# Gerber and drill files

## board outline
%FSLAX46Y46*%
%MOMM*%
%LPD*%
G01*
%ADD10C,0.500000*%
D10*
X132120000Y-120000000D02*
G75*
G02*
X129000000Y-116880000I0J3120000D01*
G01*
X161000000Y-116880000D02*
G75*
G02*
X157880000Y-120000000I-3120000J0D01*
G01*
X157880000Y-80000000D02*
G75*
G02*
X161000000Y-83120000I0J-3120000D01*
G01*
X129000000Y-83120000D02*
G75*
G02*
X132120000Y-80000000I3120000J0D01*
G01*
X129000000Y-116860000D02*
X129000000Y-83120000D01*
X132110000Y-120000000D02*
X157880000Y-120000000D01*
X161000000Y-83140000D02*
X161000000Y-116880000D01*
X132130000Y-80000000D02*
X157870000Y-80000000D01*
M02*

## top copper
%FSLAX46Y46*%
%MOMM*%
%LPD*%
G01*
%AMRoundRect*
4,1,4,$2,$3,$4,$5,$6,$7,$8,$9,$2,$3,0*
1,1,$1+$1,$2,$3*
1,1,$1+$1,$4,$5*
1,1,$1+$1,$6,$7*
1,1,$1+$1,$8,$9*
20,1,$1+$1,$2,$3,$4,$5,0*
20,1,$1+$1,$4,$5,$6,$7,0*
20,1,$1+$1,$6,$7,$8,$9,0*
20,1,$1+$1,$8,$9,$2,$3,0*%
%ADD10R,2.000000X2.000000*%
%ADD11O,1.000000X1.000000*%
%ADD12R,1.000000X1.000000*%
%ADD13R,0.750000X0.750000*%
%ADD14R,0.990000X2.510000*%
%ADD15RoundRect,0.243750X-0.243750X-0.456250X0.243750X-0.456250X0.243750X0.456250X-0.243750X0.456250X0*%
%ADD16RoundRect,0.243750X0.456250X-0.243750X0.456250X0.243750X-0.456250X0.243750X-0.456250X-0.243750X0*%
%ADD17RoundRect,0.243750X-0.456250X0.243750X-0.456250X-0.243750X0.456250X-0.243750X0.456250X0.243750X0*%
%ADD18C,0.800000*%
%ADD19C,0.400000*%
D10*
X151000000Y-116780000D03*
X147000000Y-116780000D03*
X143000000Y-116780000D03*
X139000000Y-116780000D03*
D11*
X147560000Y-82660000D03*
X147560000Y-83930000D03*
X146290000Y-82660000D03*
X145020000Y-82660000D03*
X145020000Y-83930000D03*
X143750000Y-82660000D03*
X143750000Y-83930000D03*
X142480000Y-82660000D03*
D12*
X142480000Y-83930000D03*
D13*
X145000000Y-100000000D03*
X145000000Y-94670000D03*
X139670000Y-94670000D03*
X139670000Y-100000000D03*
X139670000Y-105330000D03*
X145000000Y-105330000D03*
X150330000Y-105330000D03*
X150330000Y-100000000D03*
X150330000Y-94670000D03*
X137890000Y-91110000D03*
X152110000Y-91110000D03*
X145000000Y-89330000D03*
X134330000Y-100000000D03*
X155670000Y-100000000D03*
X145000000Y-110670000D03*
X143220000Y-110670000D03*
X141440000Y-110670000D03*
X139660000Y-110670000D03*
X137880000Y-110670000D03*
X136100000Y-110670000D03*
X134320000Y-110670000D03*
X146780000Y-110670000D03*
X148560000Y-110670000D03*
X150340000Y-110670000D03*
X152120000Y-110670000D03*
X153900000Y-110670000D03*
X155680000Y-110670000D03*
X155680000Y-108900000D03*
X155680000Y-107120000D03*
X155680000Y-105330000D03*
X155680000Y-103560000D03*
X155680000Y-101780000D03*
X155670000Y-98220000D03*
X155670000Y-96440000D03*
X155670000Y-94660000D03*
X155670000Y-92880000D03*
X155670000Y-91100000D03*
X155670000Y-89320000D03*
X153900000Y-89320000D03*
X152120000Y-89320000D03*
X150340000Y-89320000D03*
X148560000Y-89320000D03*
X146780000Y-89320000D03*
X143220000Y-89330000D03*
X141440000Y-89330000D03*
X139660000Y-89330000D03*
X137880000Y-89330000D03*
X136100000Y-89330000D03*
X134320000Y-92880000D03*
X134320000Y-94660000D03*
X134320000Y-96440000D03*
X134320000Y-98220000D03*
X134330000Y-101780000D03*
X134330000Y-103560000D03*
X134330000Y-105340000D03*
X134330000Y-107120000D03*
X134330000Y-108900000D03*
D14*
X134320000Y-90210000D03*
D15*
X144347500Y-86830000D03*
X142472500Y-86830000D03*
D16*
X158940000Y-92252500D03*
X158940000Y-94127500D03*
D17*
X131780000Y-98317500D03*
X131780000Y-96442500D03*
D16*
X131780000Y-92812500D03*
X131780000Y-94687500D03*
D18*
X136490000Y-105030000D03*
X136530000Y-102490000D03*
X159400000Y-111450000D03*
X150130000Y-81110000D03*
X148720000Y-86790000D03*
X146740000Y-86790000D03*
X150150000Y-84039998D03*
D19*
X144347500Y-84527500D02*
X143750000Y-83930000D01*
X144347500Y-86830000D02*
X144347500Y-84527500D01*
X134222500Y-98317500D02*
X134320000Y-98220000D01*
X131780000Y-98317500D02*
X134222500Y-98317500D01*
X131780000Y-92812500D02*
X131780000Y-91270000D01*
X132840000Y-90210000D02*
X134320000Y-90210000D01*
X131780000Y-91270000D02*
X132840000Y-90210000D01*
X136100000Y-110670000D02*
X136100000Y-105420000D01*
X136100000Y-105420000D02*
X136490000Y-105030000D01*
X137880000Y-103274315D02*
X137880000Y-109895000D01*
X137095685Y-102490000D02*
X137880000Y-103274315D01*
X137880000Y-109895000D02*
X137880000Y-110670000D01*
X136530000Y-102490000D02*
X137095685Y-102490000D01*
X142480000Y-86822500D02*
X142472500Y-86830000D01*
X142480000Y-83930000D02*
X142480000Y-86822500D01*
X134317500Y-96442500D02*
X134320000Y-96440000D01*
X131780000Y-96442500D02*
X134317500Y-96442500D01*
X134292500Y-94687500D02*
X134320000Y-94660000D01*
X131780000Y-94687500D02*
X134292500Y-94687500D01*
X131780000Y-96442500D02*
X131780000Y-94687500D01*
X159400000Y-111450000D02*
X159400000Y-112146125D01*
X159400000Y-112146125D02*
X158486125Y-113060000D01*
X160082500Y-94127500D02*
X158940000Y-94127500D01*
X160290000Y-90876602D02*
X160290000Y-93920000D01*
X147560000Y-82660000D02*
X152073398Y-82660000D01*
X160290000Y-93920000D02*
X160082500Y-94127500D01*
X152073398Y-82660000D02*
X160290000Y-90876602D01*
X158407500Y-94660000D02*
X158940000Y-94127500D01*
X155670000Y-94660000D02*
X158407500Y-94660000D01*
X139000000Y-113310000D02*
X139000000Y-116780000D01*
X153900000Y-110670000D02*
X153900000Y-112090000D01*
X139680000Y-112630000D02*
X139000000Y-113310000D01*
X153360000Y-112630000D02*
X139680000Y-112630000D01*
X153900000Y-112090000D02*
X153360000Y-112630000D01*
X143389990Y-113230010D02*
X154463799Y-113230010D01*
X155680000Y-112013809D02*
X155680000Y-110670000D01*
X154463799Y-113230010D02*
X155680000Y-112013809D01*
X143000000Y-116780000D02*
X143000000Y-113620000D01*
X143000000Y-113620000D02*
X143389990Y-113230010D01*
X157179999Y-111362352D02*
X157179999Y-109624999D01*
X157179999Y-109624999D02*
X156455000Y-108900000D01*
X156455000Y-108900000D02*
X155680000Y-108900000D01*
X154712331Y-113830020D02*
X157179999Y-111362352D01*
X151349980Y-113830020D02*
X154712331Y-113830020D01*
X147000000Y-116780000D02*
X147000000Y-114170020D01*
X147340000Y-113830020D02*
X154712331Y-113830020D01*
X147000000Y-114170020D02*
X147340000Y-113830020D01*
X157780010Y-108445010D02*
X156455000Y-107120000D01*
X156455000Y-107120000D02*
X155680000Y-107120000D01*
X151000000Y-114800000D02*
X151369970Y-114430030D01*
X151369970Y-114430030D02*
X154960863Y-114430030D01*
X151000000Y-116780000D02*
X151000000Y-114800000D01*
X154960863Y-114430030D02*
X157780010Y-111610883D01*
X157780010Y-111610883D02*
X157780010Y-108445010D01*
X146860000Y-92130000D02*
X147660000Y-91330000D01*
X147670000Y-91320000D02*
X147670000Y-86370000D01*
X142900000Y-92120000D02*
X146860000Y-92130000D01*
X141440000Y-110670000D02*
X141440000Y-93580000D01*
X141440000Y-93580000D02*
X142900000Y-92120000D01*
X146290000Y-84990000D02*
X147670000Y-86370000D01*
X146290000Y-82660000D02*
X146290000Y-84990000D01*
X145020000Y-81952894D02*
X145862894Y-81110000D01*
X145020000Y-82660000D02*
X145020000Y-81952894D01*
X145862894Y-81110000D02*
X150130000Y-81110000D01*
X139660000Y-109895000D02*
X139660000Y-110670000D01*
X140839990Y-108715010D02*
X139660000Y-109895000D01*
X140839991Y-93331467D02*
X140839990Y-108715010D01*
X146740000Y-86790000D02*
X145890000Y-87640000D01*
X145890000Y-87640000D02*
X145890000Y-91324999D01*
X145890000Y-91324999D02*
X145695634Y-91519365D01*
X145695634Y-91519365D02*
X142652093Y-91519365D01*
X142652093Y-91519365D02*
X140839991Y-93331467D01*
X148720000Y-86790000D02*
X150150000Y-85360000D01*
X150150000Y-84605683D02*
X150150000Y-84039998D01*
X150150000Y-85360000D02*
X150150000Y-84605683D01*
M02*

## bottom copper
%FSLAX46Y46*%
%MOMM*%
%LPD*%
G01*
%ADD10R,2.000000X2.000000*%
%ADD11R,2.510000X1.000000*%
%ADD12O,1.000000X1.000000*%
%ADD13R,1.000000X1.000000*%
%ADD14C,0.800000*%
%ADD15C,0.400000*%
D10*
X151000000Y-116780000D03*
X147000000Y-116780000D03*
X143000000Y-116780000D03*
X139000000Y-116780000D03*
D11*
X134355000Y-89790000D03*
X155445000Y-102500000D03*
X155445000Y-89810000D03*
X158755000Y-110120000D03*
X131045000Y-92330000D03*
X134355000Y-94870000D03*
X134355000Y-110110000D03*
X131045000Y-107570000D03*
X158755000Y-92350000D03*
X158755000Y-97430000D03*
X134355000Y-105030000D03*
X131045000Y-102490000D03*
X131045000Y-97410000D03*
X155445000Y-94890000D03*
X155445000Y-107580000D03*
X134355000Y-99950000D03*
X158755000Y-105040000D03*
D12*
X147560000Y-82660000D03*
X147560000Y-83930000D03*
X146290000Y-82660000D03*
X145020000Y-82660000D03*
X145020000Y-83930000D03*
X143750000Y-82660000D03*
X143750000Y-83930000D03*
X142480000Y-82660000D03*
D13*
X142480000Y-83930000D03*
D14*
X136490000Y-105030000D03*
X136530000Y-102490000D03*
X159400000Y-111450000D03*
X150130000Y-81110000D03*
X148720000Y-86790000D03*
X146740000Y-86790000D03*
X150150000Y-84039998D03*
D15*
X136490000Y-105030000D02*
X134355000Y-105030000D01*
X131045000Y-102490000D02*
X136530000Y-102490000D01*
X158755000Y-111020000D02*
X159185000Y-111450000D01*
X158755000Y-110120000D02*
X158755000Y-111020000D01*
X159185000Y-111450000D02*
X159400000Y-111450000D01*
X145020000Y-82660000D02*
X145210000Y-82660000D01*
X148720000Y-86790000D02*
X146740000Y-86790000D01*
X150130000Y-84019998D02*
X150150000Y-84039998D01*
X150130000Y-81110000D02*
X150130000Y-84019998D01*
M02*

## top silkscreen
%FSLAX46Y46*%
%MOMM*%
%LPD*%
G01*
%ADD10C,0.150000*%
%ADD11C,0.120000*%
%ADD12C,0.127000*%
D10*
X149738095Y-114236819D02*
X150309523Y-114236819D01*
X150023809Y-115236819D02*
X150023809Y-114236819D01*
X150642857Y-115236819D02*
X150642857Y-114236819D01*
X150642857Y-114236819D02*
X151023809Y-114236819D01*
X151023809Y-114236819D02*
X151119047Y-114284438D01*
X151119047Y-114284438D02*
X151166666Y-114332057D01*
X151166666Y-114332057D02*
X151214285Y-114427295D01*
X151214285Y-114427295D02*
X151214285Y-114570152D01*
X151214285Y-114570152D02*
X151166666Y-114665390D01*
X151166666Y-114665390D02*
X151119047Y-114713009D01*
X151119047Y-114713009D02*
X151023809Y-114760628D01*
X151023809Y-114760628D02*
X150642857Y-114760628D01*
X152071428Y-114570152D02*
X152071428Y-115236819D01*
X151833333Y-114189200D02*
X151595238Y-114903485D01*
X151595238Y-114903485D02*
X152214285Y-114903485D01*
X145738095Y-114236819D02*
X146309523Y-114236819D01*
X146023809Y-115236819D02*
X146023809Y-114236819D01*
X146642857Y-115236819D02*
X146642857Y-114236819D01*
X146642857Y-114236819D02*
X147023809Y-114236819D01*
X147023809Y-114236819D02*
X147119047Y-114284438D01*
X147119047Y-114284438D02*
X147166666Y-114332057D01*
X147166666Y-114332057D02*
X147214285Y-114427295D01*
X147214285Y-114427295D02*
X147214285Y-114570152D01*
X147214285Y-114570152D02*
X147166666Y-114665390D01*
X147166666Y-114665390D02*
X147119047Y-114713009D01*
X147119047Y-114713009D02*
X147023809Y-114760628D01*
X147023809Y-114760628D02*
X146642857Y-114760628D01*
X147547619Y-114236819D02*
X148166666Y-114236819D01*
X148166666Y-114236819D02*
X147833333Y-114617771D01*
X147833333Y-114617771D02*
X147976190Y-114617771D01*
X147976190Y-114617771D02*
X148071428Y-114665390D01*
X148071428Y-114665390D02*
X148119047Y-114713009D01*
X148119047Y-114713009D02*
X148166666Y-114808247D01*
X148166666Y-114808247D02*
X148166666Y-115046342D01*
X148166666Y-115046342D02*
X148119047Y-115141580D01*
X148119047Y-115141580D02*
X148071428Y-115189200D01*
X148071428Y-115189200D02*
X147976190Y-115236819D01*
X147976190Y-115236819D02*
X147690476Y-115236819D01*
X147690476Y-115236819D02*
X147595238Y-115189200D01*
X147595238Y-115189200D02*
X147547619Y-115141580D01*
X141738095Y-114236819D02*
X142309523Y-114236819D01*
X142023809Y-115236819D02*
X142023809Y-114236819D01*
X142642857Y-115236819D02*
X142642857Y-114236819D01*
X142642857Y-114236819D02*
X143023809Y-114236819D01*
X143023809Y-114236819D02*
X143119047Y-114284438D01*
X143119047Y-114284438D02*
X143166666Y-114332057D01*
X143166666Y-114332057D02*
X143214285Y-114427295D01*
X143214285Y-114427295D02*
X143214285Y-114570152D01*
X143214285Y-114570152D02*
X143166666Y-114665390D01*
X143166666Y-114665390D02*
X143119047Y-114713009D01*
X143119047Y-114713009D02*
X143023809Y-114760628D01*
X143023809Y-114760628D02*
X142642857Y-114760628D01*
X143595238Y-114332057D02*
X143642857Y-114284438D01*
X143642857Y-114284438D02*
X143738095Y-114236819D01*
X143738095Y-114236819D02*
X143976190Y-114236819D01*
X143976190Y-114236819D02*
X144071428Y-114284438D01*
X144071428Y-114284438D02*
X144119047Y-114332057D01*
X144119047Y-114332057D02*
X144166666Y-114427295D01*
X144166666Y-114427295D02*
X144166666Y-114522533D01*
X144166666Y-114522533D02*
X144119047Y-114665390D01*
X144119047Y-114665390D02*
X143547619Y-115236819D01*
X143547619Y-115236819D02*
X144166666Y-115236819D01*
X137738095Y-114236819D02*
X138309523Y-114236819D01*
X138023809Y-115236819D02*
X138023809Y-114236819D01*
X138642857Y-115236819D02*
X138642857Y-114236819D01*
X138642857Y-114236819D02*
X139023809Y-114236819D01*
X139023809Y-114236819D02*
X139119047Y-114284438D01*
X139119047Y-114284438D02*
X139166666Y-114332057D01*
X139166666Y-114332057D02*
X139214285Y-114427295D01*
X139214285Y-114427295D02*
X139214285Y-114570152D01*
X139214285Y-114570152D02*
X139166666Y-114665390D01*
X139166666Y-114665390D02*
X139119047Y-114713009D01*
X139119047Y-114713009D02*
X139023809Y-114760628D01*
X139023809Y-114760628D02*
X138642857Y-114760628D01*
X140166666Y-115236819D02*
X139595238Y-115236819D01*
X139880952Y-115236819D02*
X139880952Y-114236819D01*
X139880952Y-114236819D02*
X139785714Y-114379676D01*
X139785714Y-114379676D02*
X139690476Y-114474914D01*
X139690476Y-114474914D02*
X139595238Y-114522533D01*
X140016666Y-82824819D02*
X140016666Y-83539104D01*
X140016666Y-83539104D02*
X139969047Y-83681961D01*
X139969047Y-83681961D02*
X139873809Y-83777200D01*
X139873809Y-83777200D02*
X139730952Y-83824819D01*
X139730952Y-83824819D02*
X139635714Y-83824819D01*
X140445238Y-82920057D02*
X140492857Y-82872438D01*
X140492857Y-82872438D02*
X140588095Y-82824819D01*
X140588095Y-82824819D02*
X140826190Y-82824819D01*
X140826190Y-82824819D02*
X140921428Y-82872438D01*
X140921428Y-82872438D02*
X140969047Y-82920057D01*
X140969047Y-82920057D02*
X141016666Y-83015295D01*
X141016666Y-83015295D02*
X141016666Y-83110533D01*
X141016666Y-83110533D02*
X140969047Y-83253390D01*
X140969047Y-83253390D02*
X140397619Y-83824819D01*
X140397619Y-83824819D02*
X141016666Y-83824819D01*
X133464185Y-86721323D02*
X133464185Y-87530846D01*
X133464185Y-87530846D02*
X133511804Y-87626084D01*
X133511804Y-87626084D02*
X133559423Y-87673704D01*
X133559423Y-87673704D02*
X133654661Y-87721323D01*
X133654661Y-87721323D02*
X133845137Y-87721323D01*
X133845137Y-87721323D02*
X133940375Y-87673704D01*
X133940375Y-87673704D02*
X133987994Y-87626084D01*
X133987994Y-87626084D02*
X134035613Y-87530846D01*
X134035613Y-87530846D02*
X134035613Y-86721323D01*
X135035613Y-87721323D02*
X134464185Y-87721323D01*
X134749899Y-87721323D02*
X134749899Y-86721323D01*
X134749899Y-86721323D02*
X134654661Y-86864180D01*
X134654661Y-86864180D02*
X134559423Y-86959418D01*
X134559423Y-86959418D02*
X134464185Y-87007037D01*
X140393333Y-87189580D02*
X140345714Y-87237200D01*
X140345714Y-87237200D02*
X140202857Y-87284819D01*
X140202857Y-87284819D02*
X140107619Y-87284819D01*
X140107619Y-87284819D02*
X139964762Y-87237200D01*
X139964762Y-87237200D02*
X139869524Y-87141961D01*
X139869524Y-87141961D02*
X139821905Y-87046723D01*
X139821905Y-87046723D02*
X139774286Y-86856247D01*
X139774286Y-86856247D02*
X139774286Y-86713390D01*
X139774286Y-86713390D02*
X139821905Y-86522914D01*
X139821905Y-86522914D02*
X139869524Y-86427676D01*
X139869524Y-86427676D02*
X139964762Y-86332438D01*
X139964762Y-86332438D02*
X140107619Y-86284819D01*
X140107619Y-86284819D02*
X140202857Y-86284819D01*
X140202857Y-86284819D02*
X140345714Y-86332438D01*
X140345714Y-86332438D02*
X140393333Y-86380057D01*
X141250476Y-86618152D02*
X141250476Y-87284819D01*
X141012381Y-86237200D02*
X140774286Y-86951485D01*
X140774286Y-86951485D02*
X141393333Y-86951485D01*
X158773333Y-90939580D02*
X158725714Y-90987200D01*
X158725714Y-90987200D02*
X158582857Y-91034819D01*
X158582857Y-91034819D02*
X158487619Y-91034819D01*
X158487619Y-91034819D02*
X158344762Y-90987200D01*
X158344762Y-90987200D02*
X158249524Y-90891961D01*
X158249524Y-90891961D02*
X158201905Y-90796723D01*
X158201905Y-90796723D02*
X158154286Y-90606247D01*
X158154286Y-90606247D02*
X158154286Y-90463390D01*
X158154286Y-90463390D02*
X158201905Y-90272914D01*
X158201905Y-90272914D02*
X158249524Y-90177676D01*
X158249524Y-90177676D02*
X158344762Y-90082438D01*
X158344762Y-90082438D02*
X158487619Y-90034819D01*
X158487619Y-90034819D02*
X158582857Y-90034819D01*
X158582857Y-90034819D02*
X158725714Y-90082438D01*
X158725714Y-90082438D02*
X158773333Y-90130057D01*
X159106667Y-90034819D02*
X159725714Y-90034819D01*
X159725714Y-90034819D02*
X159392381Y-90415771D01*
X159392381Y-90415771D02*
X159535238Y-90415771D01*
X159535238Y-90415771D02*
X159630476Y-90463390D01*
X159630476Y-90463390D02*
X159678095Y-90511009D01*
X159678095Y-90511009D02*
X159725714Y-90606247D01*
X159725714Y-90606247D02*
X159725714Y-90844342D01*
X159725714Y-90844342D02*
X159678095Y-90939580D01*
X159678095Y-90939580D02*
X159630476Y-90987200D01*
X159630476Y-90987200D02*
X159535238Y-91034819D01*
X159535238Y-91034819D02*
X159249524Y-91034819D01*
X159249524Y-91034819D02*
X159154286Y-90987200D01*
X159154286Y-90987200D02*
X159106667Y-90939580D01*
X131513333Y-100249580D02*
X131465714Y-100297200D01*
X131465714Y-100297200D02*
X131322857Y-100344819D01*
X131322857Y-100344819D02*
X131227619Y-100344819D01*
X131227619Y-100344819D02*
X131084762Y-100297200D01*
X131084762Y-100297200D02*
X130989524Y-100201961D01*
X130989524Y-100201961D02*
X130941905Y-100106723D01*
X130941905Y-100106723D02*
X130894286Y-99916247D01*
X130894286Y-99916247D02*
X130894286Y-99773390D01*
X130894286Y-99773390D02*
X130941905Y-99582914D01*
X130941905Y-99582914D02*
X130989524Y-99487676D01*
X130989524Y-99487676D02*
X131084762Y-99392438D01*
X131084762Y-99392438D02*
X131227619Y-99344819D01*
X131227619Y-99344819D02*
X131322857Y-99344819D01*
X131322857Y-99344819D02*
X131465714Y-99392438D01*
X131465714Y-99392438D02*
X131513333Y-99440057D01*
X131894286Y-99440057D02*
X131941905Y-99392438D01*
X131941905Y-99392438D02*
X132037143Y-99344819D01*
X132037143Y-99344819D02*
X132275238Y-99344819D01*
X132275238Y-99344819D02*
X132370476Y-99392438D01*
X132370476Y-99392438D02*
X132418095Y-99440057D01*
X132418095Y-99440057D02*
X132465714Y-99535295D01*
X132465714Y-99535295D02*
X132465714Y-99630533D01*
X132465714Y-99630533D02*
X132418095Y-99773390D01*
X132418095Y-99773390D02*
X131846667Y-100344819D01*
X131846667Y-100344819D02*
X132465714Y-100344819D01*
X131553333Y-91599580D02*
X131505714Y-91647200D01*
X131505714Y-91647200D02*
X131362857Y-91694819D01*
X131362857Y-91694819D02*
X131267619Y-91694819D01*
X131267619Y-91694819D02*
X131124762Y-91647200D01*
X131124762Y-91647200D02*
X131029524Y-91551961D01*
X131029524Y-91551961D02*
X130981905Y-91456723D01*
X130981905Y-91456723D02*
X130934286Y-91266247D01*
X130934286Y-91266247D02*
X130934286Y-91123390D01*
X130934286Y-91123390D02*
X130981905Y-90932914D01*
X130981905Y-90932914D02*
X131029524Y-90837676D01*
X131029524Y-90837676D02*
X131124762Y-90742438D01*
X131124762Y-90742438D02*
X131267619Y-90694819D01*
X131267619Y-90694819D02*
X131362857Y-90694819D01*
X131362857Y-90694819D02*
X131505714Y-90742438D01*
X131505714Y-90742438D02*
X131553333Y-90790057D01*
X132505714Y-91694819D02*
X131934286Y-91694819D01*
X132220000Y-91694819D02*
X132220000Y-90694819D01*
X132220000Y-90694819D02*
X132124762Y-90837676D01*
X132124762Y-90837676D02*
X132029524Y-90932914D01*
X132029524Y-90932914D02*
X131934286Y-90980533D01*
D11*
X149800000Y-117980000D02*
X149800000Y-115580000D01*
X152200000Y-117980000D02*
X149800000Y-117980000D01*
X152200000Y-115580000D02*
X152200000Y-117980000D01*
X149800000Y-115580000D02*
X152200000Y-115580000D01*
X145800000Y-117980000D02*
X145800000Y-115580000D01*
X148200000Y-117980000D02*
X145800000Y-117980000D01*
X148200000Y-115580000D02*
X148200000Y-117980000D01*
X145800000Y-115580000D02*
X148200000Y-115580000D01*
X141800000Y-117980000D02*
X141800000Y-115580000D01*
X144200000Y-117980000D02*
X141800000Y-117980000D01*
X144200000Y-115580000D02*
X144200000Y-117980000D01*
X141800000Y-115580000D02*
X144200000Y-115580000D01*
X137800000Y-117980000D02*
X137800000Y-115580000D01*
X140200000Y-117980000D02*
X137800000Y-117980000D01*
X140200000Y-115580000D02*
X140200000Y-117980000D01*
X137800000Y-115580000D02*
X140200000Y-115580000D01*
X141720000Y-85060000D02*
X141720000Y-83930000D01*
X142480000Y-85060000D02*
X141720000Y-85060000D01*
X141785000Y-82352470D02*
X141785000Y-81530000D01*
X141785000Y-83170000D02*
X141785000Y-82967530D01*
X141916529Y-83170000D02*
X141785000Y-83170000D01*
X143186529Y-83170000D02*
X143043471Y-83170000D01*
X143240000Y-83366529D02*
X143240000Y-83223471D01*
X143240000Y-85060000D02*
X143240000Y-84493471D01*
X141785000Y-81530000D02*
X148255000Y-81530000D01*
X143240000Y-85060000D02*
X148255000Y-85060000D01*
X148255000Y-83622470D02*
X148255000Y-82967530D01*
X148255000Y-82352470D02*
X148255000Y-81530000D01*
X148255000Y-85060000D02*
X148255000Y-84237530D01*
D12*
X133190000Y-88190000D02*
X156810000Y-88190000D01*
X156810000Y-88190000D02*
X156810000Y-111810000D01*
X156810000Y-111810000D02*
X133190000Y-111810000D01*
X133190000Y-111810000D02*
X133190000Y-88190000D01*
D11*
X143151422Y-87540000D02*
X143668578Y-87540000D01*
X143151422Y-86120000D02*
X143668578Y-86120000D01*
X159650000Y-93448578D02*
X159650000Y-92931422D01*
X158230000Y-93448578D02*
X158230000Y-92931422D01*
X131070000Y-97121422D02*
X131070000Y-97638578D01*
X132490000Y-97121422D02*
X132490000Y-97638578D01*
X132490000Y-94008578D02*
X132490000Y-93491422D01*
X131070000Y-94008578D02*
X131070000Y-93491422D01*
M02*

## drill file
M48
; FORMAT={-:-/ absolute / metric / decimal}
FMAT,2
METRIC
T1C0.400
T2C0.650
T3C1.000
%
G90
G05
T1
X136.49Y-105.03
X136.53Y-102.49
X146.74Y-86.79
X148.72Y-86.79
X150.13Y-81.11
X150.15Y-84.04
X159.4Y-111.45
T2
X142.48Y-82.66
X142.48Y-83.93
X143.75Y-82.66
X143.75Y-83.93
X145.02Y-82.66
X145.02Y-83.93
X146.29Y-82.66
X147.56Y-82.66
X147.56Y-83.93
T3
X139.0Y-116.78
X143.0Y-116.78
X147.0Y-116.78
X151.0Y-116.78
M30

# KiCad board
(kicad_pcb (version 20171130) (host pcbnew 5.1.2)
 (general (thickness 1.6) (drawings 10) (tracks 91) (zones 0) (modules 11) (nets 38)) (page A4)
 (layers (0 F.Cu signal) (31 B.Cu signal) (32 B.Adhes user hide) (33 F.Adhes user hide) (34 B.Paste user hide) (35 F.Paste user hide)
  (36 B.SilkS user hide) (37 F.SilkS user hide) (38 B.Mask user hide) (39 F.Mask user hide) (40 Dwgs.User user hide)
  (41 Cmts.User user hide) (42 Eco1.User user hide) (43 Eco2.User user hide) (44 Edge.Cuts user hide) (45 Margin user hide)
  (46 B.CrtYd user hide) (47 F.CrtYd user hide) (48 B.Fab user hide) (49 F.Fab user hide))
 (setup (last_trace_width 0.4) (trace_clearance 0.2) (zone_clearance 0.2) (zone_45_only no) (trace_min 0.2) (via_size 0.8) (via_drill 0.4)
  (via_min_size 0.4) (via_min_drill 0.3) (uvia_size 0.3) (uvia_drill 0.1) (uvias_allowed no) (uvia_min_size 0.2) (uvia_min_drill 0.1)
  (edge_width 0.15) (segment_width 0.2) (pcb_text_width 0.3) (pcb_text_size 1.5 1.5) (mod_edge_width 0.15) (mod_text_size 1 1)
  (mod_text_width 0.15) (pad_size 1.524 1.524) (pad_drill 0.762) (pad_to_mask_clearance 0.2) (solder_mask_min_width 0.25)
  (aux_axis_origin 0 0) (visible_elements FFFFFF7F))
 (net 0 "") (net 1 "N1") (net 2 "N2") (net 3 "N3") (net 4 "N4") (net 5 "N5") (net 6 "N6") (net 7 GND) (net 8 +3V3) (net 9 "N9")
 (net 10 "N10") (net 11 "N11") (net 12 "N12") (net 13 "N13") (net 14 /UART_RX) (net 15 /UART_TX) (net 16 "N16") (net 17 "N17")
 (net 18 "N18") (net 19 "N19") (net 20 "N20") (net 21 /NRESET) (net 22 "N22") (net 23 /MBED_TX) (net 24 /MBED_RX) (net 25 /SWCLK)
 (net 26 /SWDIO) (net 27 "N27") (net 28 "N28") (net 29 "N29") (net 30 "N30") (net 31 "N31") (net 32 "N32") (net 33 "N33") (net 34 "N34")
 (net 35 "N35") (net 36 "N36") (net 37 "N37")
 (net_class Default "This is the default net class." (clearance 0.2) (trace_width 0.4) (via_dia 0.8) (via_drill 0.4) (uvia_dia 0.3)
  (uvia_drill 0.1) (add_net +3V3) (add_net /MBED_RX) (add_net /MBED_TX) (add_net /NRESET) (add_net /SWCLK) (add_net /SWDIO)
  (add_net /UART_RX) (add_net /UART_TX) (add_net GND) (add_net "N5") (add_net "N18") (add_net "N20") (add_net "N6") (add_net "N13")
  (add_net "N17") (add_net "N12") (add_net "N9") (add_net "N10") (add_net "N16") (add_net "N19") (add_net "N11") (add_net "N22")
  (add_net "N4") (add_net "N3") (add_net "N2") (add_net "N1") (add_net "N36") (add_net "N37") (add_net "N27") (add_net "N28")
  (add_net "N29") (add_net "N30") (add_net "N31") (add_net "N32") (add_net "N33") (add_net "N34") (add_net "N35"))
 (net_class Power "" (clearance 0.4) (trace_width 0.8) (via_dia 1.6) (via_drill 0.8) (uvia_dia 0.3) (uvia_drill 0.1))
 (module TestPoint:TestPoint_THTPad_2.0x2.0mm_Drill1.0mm (layer F.Cu) (at 151 116.78)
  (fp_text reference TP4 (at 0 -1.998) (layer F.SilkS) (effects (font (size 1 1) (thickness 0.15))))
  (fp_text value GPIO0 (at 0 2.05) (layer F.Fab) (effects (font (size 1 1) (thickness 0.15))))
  (fp_line (start -1.2 1.2) (end -1.2 -1.2) (layer F.SilkS) (width 0.12))
  (fp_line (start 1.2 1.2) (end -1.2 1.2) (layer F.SilkS) (width 0.12))
  (fp_line (start 1.2 -1.2) (end 1.2 1.2) (layer F.SilkS) (width 0.12))
  (fp_line (start -1.2 -1.2) (end 1.2 -1.2) (layer F.SilkS) (width 0.12))
  (pad 1 thru_hole rect (at 0 0) (size 2 2) (drill 1) (layers *.Cu *.Mask) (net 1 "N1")))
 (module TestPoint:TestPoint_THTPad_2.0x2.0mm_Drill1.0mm (layer F.Cu) (at 147 116.78)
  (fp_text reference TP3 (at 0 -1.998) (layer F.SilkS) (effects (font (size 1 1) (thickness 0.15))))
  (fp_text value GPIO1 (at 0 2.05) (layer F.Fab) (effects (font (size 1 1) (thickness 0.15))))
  (fp_line (start -1.2 1.2) (end -1.2 -1.2) (layer F.SilkS) (width 0.12))
  (fp_line (start 1.2 1.2) (end -1.2 1.2) (layer F.SilkS) (width 0.12))
  (fp_line (start 1.2 -1.2) (end 1.2 1.2) (layer F.SilkS) (width 0.12))
  (fp_line (start -1.2 -1.2) (end 1.2 -1.2) (layer F.SilkS) (width 0.12))
  (pad 1 thru_hole rect (at 0 0) (size 2 2) (drill 1) (layers *.Cu *.Mask) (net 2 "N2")))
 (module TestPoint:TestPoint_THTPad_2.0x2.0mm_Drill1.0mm (layer F.Cu) (at 143 116.78)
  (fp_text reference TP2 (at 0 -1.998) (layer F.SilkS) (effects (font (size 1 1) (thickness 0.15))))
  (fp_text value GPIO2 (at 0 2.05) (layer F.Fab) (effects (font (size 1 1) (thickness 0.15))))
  (fp_line (start -1.2 1.2) (end -1.2 -1.2) (layer F.SilkS) (width 0.12))
  (fp_line (start 1.2 1.2) (end -1.2 1.2) (layer F.SilkS) (width 0.12))
  (fp_line (start 1.2 -1.2) (end 1.2 1.2) (layer F.SilkS) (width 0.12))
  (fp_line (start -1.2 -1.2) (end 1.2 -1.2) (layer F.SilkS) (width 0.12))
  (pad 1 thru_hole rect (at 0 0) (size 2 2) (drill 1) (layers *.Cu *.Mask) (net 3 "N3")))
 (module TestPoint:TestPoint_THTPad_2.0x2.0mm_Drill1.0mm (layer F.Cu) (at 139 116.78)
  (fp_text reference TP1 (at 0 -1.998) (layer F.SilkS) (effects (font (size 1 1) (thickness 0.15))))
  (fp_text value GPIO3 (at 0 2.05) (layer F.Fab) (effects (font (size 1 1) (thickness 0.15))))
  (fp_line (start -1.2 1.2) (end -1.2 -1.2) (layer F.SilkS) (width 0.12))
  (fp_line (start 1.2 1.2) (end -1.2 1.2) (layer F.SilkS) (width 0.12))
  (fp_line (start 1.2 -1.2) (end 1.2 1.2) (layer F.SilkS) (width 0.12))
  (fp_line (start -1.2 -1.2) (end 1.2 -1.2) (layer F.SilkS) (width 0.12))
  (pad 1 thru_hole rect (at 0 0) (size 2 2) (drill 1) (layers *.Cu *.Mask) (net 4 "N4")))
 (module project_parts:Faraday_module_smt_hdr (layer B.Cu) (at 145 100 180)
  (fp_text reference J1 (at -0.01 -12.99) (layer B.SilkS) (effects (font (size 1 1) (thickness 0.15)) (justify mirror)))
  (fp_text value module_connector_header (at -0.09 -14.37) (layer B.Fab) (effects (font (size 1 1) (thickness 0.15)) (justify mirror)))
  (pad 1 smd rect (at 10.645 10.21 180) (size 2.51 1) (layers B.Cu B.Paste B.Mask) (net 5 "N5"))
  (pad 13 smd rect (at -10.445 -2.5 180) (size 2.51 1) (layers B.Cu B.Paste B.Mask) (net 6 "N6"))
  (pad 17 smd rect (at -10.445 10.19 180) (size 2.51 1) (layers B.Cu B.Paste B.Mask) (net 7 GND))
  (pad 10 smd rect (at -13.755 -10.12 180) (size 2.51 1) (layers B.Cu B.Paste B.Mask) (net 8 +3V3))
  (pad 2 smd rect (at 13.955 7.67 180) (size 2.51 1) (layers B.Cu B.Paste B.Mask) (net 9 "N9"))
  (pad 3 smd rect (at 10.645 5.13 180) (size 2.51 1) (layers B.Cu B.Paste B.Mask) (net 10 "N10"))
  (pad 9 smd rect (at 10.645 -10.11 180) (size 2.51 1) (layers B.Cu B.Paste B.Mask) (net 7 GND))
  (pad 8 smd rect (at 13.955 -7.57 180) (size 2.51 1) (layers B.Cu B.Paste B.Mask) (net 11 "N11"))
  (pad 16 smd rect (at -13.755 7.65 180) (size 2.51 1) (layers B.Cu B.Paste B.Mask) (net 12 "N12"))
  (pad 14 smd rect (at -13.755 2.57 180) (size 2.51 1) (layers B.Cu B.Paste B.Mask) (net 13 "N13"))
  (pad 7 smd rect (at 10.645 -5.03 180) (size 2.51 1) (layers B.Cu B.Paste B.Mask) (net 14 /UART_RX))
  (pad 6 smd rect (at 13.955 -2.49 180) (size 2.51 1) (layers B.Cu B.Paste B.Mask) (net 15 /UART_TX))
  (pad 4 smd rect (at 13.955 2.59 180) (size 2.51 1) (layers B.Cu B.Paste B.Mask) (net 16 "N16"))
  (pad 15 smd rect (at -10.445 5.11 180) (size 2.51 1) (layers B.Cu B.Paste B.Mask) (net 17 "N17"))
  (pad 11 smd rect (at -10.445 -7.58 180) (size 2.51 1) (layers B.Cu B.Paste B.Mask) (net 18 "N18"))
  (pad 5 smd rect (at 10.645 0.05 180) (size 2.51 1) (layers B.Cu B.Paste B.Mask) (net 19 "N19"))
  (pad 12 smd rect (at -13.755 -5.04 180) (size 2.51 1) (layers B.Cu B.Paste B.Mask) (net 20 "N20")))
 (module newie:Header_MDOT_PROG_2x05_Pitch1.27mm (layer F.Cu) (at 142.48 83.93 90)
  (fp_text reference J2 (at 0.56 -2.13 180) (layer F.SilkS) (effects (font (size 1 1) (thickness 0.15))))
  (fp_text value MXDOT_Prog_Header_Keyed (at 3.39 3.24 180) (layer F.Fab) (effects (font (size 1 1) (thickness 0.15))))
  (fp_line (start -1.13 -0.76) (end 0 -0.76) (layer F.SilkS) (width 0.12))
  (fp_line (start -1.13 0) (end -1.13 -0.76) (layer F.SilkS) (width 0.12))
  (fp_line (start 1.57753 -0.695) (end 2.4 -0.695) (layer F.SilkS) (width 0.12))
  (fp_line (start 0.76 -0.695) (end 0.96247 -0.695) (layer F.SilkS) (width 0.12))
  (fp_line (start 0.76 -0.563471) (end 0.76 -0.695) (layer F.SilkS) (width 0.12))
  (fp_line (start 0.76 0.706529) (end 0.76 0.563471) (layer F.SilkS) (width 0.12))
  (fp_line (start 0.563471 0.76) (end 0.706529 0.76) (layer F.SilkS) (width 0.12))
  (fp_line (start -1.13 0.76) (end -0.563471 0.76) (layer F.SilkS) (width 0.12))
  (fp_line (start 2.4 -0.695) (end 2.4 5.775) (layer F.SilkS) (width 0.12))
  (fp_line (start -1.13 0.76) (end -1.13 5.775) (layer F.SilkS) (width 0.12))
  (fp_line (start 0.30753 5.775) (end 0.96247 5.775) (layer F.SilkS) (width 0.12))
  (fp_line (start 1.57753 5.775) (end 2.4 5.775) (layer F.SilkS) (width 0.12))
  (fp_line (start -1.13 5.775) (end -0.30753 5.775) (layer F.SilkS) (width 0.12))
  (pad 10 thru_hole oval (at 1.27 5.08 90) (size 1 1) (drill 0.65) (layers *.Cu *.Mask) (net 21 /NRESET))
  (pad 9 thru_hole oval (at 0 5.08 90) (size 1 1) (drill 0.65) (layers *.Cu *.Mask) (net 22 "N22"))
  (pad 8 thru_hole oval (at 1.27 3.81 90) (size 1 1) (drill 0.65) (layers *.Cu *.Mask) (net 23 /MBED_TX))
  (pad 6 thru_hole oval (at 1.27 2.54 90) (size 1 1) (drill 0.65) (layers *.Cu *.Mask) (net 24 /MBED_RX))
  (pad 5 thru_hole oval (at 0 2.54 90) (size 1 1) (drill 0.65) (layers *.Cu *.Mask) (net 7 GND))
  (pad 4 thru_hole oval (at 1.27 1.27 90) (size 1 1) (drill 0.65) (layers *.Cu *.Mask) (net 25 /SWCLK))
  (pad 3 thru_hole oval (at 0 1.27 90) (size 1 1) (drill 0.65) (layers *.Cu *.Mask) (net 7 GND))
  (pad 2 thru_hole oval (at 1.27 0 90) (size 1 1) (drill 0.65) (layers *.Cu *.Mask) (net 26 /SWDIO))
  (pad 1 thru_hole rect (at 0 0 90) (size 1 1) (drill 0.65) (layers *.Cu *.Mask) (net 8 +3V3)))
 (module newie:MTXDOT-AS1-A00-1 (layer F.Cu) (at 145 100)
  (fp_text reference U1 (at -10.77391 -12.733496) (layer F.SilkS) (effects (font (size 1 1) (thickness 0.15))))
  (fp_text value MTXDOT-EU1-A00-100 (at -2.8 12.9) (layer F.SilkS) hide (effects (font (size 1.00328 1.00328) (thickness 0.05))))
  (fp_line (start -11.81 -11.81) (end 11.81 -11.81) (layer F.SilkS) (width 0.127))
  (fp_line (start 11.81 -11.81) (end 11.81 11.81) (layer F.SilkS) (width 0.127))
  (fp_line (start 11.81 11.81) (end -11.81 11.81) (layer F.SilkS) (width 0.127))
  (fp_line (start -11.81 11.81) (end -11.81 -11.81) (layer F.SilkS) (width 0.127))
  (pad 54 smd rect (at 0 0) (size 0.75 0.75) (layers F.Cu F.Paste F.Mask) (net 7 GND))
  (pad 51 smd rect (at 0 -5.33) (size 0.75 0.75) (layers F.Cu F.Paste F.Mask) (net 7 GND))
  (pad 50 smd rect (at -5.33 -5.33) (size 0.75 0.75) (layers F.Cu F.Paste F.Mask) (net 7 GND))
  (pad 53 smd rect (at -5.33 0) (size 0.75 0.75) (layers F.Cu F.Paste F.Mask) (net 7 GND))
  (pad 56 smd rect (at -5.33 5.33) (size 0.75 0.75) (layers F.Cu F.Paste F.Mask) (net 7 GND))
  (pad 57 smd rect (at 0 5.33) (size 0.75 0.75) (layers F.Cu F.Paste F.Mask) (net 7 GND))
  (pad 58 smd rect (at 5.33 5.33) (size 0.75 0.75) (layers F.Cu F.Paste F.Mask) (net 7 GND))
  (pad 55 smd rect (at 5.33 0) (size 0.75 0.75) (layers F.Cu F.Paste F.Mask) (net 7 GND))
  (pad 52 smd rect (at 5.33 -5.33) (size 0.75 0.75) (layers F.Cu F.Paste F.Mask) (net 7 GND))
  (pad 49 smd rect (at -7.11 -8.89) (size 0.75 0.75) (layers F.Cu F.Paste F.Mask) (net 7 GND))
  (pad 48 smd rect (at 7.11 -8.89) (size 0.75 0.75) (layers F.Cu F.Paste F.Mask) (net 7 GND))
  (pad 42 smd rect (at 0 -10.67) (size 0.75 0.75) (layers F.Cu F.Paste F.Mask) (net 7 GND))
  (pad 6 smd rect (at -10.67 0) (size 0.75 0.75) (layers F.Cu F.Paste F.Mask))
  (pad 30 smd rect (at 10.67 0) (size 0.75 0.75) (layers F.Cu F.Paste F.Mask) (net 26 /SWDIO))
  (pad 18 smd rect (at 0 10.67) (size 0.75 0.75) (layers F.Cu F.Paste F.Mask))
  (pad 17 smd rect (at -1.78 10.67) (size 0.75 0.75) (layers F.Cu F.Paste F.Mask) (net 7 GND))
  (pad 16 smd rect (at -3.56 10.67) (size 0.75 0.75) (layers F.Cu F.Paste F.Mask) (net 23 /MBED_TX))
  (pad 15 smd rect (at -5.34 10.67) (size 0.75 0.75) (layers F.Cu F.Paste F.Mask) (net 24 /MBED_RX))
  (pad 14 smd rect (at -7.12 10.67) (size 0.75 0.75) (layers F.Cu F.Paste F.Mask) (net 15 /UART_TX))
  (pad 13 smd rect (at -8.9 10.67) (size 0.75 0.75) (layers F.Cu F.Paste F.Mask) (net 14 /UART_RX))
  (pad 12 smd rect (at -10.68 10.67) (size 0.75 0.75) (layers F.Cu F.Paste F.Mask) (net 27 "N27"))
  (pad 19 smd rect (at 1.78 10.67) (size 0.75 0.75) (layers F.Cu F.Paste F.Mask))
  (pad 20 smd rect (at 3.56 10.67) (size 0.75 0.75) (layers F.Cu F.Paste F.Mask) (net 7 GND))
  (pad 21 smd rect (at 5.34 10.67) (size 0.75 0.75) (layers F.Cu F.Paste F.Mask))
  (pad 22 smd rect (at 7.12 10.67) (size 0.75 0.75) (layers F.Cu F.Paste F.Mask))
  (pad 23 smd rect (at 8.9 10.67) (size 0.75 0.75) (layers F.Cu F.Paste F.Mask) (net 4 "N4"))
  (pad 24 smd rect (at 10.68 10.67) (size 0.75 0.75) (layers F.Cu F.Paste F.Mask) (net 3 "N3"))
  (pad 25 smd rect (at 10.68 8.9) (size 0.75 0.75) (layers F.Cu F.Paste F.Mask) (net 2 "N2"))
  (pad 26 smd rect (at 10.68 7.12) (size 0.75 0.75) (layers F.Cu F.Paste F.Mask) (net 1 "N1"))
  (pad 27 smd rect (at 10.68 5.33) (size 0.75 0.75) (layers F.Cu F.Paste F.Mask) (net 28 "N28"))
  (pad 28 smd rect (at 10.68 3.56) (size 0.75 0.75) (layers F.Cu F.Paste F.Mask) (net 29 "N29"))
  (pad 29 smd rect (at 10.68 1.78) (size 0.75 0.75) (layers F.Cu F.Paste F.Mask) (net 25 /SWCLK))
  (pad 31 smd rect (at 10.67 -1.78) (size 0.75 0.75) (layers F.Cu F.Paste F.Mask) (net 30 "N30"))
  (pad 32 smd rect (at 10.67 -3.56) (size 0.75 0.75) (layers F.Cu F.Paste F.Mask) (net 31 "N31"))
  (pad 33 smd rect (at 10.67 -5.34) (size 0.75 0.75) (layers F.Cu F.Paste F.Mask) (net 21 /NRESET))
  (pad 34 smd rect (at 10.67 -7.12) (size 0.75 0.75) (layers F.Cu F.Paste F.Mask) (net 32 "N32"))
  (pad 35 smd rect (at 10.67 -8.9) (size 0.75 0.75) (layers F.Cu F.Paste F.Mask) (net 7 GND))
  (pad 36 smd rect (at 10.67 -10.68) (size 0.75 0.75) (layers F.Cu F.Paste F.Mask) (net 7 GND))
  (pad 37 smd rect (at 8.9 -10.68) (size 0.75 0.75) (layers F.Cu F.Paste F.Mask) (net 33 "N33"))
  (pad 38 smd rect (at 7.12 -10.68) (size 0.75 0.75) (layers F.Cu F.Paste F.Mask) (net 7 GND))
  (pad 39 smd rect (at 5.34 -10.68) (size 0.75 0.75) (layers F.Cu F.Paste F.Mask) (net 7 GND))
  (pad 40 smd rect (at 3.56 -10.68) (size 0.75 0.75) (layers F.Cu F.Paste F.Mask) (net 7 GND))
  (pad 41 smd rect (at 1.78 -10.68) (size 0.75 0.75) (layers F.Cu F.Paste F.Mask) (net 7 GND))
  (pad 43 smd rect (at -1.78 -10.67) (size 0.75 0.75) (layers F.Cu F.Paste F.Mask) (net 7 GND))
  (pad 44 smd rect (at -3.56 -10.67) (size 0.75 0.75) (layers F.Cu F.Paste F.Mask) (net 7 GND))
  (pad 45 smd rect (at -5.34 -10.67) (size 0.75 0.75) (layers F.Cu F.Paste F.Mask) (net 7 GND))
  (pad 46 smd rect (at -7.12 -10.67) (size 0.75 0.75) (layers F.Cu F.Paste F.Mask) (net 7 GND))
  (pad 47 smd rect (at -8.9 -10.67) (size 0.75 0.75) (layers F.Cu F.Paste F.Mask) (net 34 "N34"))
  (pad 2 smd rect (at -10.68 -7.12) (size 0.75 0.75) (layers F.Cu F.Paste F.Mask))
  (pad 3 smd rect (at -10.68 -5.34) (size 0.75 0.75) (layers F.Cu F.Paste F.Mask) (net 8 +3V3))
  (pad 4 smd rect (at -10.68 -3.56) (size 0.75 0.75) (layers F.Cu F.Paste F.Mask) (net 8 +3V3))
  (pad 5 smd rect (at -10.68 -1.78) (size 0.75 0.75) (layers F.Cu F.Paste F.Mask) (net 7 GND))
  (pad 7 smd rect (at -10.67 1.78) (size 0.75 0.75) (layers F.Cu F.Paste F.Mask))
  (pad 8 smd rect (at -10.67 3.56) (size 0.75 0.75) (layers F.Cu F.Paste F.Mask))
  (pad 9 smd rect (at -10.67 5.34) (size 0.75 0.75) (layers F.Cu F.Paste F.Mask) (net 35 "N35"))
  (pad 10 smd rect (at -10.67 7.12) (size 0.75 0.75) (layers F.Cu F.Paste F.Mask) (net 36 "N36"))
  (pad 11 smd rect (at -10.67 8.9) (size 0.75 0.75) (layers F.Cu F.Paste F.Mask) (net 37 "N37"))
  (pad 1 smd rect (at -10.68 -9.79) (size 0.99 2.51) (layers F.Cu F.Paste F.Mask) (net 7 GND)))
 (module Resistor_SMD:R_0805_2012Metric (layer F.Cu) (at 143.41 86.83)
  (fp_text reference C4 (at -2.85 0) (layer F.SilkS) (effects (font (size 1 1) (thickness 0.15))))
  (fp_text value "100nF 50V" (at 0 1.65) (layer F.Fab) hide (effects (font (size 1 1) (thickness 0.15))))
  (fp_line (start -0.258578 0.71) (end 0.258578 0.71) (layer F.SilkS) (width 0.12))
  (fp_line (start -0.258578 -0.71) (end 0.258578 -0.71) (layer F.SilkS) (width 0.12))
  (pad 2 smd roundrect (at 0.9375 0) (size 0.975 1.4) (layers F.Cu F.Paste F.Mask) (roundrect_rratio 0.25) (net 7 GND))
  (pad 1 smd roundrect (at -0.9375 0) (size 0.975 1.4) (layers F.Cu F.Paste F.Mask) (roundrect_rratio 0.25) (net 8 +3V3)))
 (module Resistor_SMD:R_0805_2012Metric (layer F.Cu) (at 158.94 93.19 90)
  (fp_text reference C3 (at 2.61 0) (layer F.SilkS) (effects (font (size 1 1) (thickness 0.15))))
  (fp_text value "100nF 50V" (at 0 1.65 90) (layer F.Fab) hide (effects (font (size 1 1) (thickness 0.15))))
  (fp_line (start -0.258578 0.71) (end 0.258578 0.71) (layer F.SilkS) (width 0.12))
  (fp_line (start -0.258578 -0.71) (end 0.258578 -0.71) (layer F.SilkS) (width 0.12))
  (pad 2 smd roundrect (at 0.9375 0 90) (size 0.975 1.4) (layers F.Cu F.Paste F.Mask) (roundrect_rratio 0.25) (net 7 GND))
  (pad 1 smd roundrect (at -0.9375 0 90) (size 0.975 1.4) (layers F.Cu F.Paste F.Mask) (roundrect_rratio 0.25) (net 21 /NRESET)))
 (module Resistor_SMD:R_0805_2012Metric (layer F.Cu) (at 131.78 97.38 270)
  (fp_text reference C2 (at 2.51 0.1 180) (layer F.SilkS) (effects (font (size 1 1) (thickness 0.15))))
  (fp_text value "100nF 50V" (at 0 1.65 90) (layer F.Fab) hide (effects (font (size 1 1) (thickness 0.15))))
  (fp_line (start -0.258578 0.71) (end 0.258578 0.71) (layer F.SilkS) (width 0.12))
  (fp_line (start -0.258578 -0.71) (end 0.258578 -0.71) (layer F.SilkS) (width 0.12))
  (pad 2 smd roundrect (at 0.9375 0 270) (size 0.975 1.4) (layers F.Cu F.Paste F.Mask) (roundrect_rratio 0.25) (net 7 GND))
  (pad 1 smd roundrect (at -0.9375 0 270) (size 0.975 1.4) (layers F.Cu F.Paste F.Mask) (roundrect_rratio 0.25) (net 8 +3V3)))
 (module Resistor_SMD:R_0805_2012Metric (layer F.Cu) (at 131.78 93.75 90)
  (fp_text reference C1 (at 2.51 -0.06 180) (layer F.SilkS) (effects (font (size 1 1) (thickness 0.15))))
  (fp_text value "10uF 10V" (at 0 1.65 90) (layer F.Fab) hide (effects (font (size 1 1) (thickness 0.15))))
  (fp_line (start -0.258578 0.71) (end 0.258578 0.71) (layer F.SilkS) (width 0.12))
  (fp_line (start -0.258578 -0.71) (end 0.258578 -0.71) (layer F.SilkS) (width 0.12))
  (pad 2 smd roundrect (at 0.9375 0 90) (size 0.975 1.4) (layers F.Cu F.Paste F.Mask) (roundrect_rratio 0.25) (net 7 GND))
  (pad 1 smd roundrect (at -0.9375 0 90) (size 0.975 1.4) (layers F.Cu F.Paste F.Mask) (roundrect_rratio 0.25) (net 8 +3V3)))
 (gr_arc (start 132.12 116.88) (end 129 116.88) (angle -90) (layer Edge.Cuts) (width 0.5))
 (gr_arc (start 157.88 116.88) (end 157.88 120) (angle -90) (layer Edge.Cuts) (width 0.5))
 (gr_arc (start 157.88 83.12) (end 157.88 80) (angle 90) (layer Edge.Cuts) (width 0.5))
 (gr_arc (start 132.12 83.12) (end 132.12 80) (angle -90) (layer Edge.Cuts) (width 0.5))
 (gr_line (start 129 116.86) (end 129 83.12) (layer Edge.Cuts) (width 0.5))
 (gr_line (start 132.11 120) (end 157.88 120) (layer Edge.Cuts) (width 0.5))
 (gr_line (start 161 83.14) (end 161 116.88) (layer Edge.Cuts) (width 0.5))
 (gr_line (start 132.13 80) (end 157.87 80) (layer Edge.Cuts) (width 0.5))
 (segment (start 144.3475 84.5275) (end 143.75 83.93) (width 0.4) (layer F.Cu) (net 7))
 (segment (start 144.3475 86.83) (end 144.3475 84.5275) (width 0.4) (layer F.Cu) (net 7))
 (segment (start 134.2225 98.3175) (end 134.32 98.22) (width 0.4) (layer F.Cu) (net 7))
 (segment (start 131.78 98.3175) (end 134.2225 98.3175) (width 0.4) (layer F.Cu) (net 7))
 (segment (start 131.78 92.8125) (end 131.78 91.27) (width 0.4) (layer F.Cu) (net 7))
 (segment (start 132.84 90.21) (end 134.32 90.21) (width 0.4) (layer F.Cu) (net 7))
 (segment (start 131.78 91.27) (end 132.84 90.21) (width 0.4) (layer F.Cu) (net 7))
 (segment (start 136.1 110.67) (end 136.1 105.42) (width 0.4) (layer F.Cu) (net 14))
 (via (at 136.49 105.03) (size 0.8) (drill 0.4) (layers F.Cu B.Cu) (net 14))
 (segment (start 136.1 105.42) (end 136.49 105.03) (width 0.4) (layer F.Cu) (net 14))
 (segment (start 136.49 105.03) (end 134.355 105.03) (width 0.4) (layer B.Cu) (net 14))
 (segment (start 131.045 102.49) (end 136.53 102.49) (width 0.4) (layer B.Cu) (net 15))
 (via (at 136.53 102.49) (size 0.8) (drill 0.4) (layers F.Cu B.Cu) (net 15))
 (segment (start 137.88 103.274315) (end 137.88 109.895) (width 0.4) (layer F.Cu) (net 15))
 (segment (start 137.095685 102.49) (end 137.88 103.274315) (width 0.4) (layer F.Cu) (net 15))
 (segment (start 137.88 109.895) (end 137.88 110.67) (width 0.4) (layer F.Cu) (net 15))
 (segment (start 136.53 102.49) (end 137.095685 102.49) (width 0.4) (layer F.Cu) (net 15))
 (segment (start 142.48 86.8225) (end 142.4725 86.83) (width 0.4) (layer F.Cu) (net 8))
 (segment (start 142.48 83.93) (end 142.48 86.8225) (width 0.4) (layer F.Cu) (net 8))
 (segment (start 134.3175 96.4425) (end 134.32 96.44) (width 0.4) (layer F.Cu) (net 8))
 (segment (start 131.78 96.4425) (end 134.3175 96.4425) (width 0.4) (layer F.Cu) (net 8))
 (segment (start 134.2925 94.6875) (end 134.32 94.66) (width 0.4) (layer F.Cu) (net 8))
 (segment (start 131.78 94.6875) (end 134.2925 94.6875) (width 0.4) (layer F.Cu) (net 8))
 (segment (start 131.78 96.4425) (end 131.78 94.6875) (width 0.4) (layer F.Cu) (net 8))
 (segment (start 158.755 111.02) (end 159.185 111.45) (width 0.4) (layer B.Cu) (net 8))
 (segment (start 158.755 110.12) (end 158.755 111.02) (width 0.4) (layer B.Cu) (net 8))
 (via (at 159.4 111.45) (size 0.8) (drill 0.4) (layers F.Cu B.Cu) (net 8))
 (segment (start 159.185 111.45) (end 159.4 111.45) (width 0.4) (layer B.Cu) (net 8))
 (segment (start 159.4 111.45) (end 159.4 112.146125) (width 0.4) (layer F.Cu) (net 8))
 (segment (start 159.4 112.146125) (end 158.486125 113.06) (width 0.4) (layer F.Cu) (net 8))
 (segment (start 160.0825 94.1275) (end 158.94 94.1275) (width 0.4) (layer F.Cu) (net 21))
 (segment (start 160.29 90.876602) (end 160.29 93.92) (width 0.4) (layer F.Cu) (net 21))
 (segment (start 147.56 82.66) (end 152.073398 82.66) (width 0.4) (layer F.Cu) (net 21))
 (segment (start 160.29 93.92) (end 160.0825 94.1275) (width 0.4) (layer F.Cu) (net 21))
 (segment (start 152.073398 82.66) (end 160.29 90.876602) (width 0.4) (layer F.Cu) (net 21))
 (segment (start 158.4075 94.66) (end 158.94 94.1275) (width 0.4) (layer F.Cu) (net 21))
 (segment (start 155.67 94.66) (end 158.4075 94.66) (width 0.4) (layer F.Cu) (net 21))
 (segment (start 139 113.31) (end 139 116.78) (width 0.4) (layer F.Cu) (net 4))
 (segment (start 153.9 110.67) (end 153.9 112.09) (width 0.4) (layer F.Cu) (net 4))
 (segment (start 139.68 112.63) (end 139 113.31) (width 0.4) (layer F.Cu) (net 4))
 (segment (start 153.36 112.63) (end 139.68 112.63) (width 0.4) (layer F.Cu) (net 4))
 (segment (start 153.9 112.09) (end 153.36 112.63) (width 0.4) (layer F.Cu) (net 4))
 (segment (start 143.38999 113.23001) (end 154.463799 113.23001) (width 0.4) (layer F.Cu) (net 3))
 (segment (start 155.68 112.013809) (end 155.68 110.67) (width 0.4) (layer F.Cu) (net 3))
 (segment (start 154.463799 113.23001) (end 155.68 112.013809) (width 0.4) (layer F.Cu) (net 3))
 (segment (start 143 116.78) (end 143 113.62) (width 0.4) (layer F.Cu) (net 3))
 (segment (start 143 113.62) (end 143.38999 113.23001) (width 0.4) (layer F.Cu) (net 3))
 (segment (start 157.179999 111.362352) (end 157.179999 109.624999) (width 0.4) (layer F.Cu) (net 2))
 (segment (start 157.179999 109.624999) (end 156.455 108.9) (width 0.4) (layer F.Cu) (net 2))
 (segment (start 156.455 108.9) (end 155.68 108.9) (width 0.4) (layer F.Cu) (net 2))
 (segment (start 154.712331 113.83002) (end 157.179999 111.362352) (width 0.4) (layer F.Cu) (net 2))
 (segment (start 151.34998 113.83002) (end 154.712331 113.83002) (width 0.4) (layer F.Cu) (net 2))
 (segment (start 147 116.78) (end 147 114.17002) (width 0.4) (layer F.Cu) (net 2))
 (segment (start 147.34 113.83002) (end 154.712331 113.83002) (width 0.4) (layer F.Cu) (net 2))
 (segment (start 147 114.17002) (end 147.34 113.83002) (width 0.4) (layer F.Cu) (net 2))
 (segment (start 157.78001 108.44501) (end 156.455 107.12) (width 0.4) (layer F.Cu) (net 1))
 (segment (start 156.455 107.12) (end 155.68 107.12) (width 0.4) (layer F.Cu) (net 1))
 (segment (start 151 114.8) (end 151.36997 114.43003) (width 0.4) (layer F.Cu) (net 1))
 (segment (start 151.36997 114.43003) (end 154.960863 114.43003) (width 0.4) (layer F.Cu) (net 1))
 (segment (start 151 116.78) (end 151 114.8) (width 0.4) (layer F.Cu) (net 1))
 (segment (start 154.960863 114.43003) (end 157.78001 111.610883) (width 0.4) (layer F.Cu) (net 1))
 (segment (start 157.78001 111.610883) (end 157.78001 108.44501) (width 0.4) (layer F.Cu) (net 1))
 (segment (start 146.86 92.13) (end 147.66 91.33) (width 0.4) (layer F.Cu) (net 23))
 (segment (start 147.67 91.32) (end 147.67 86.37) (width 0.4) (layer F.Cu) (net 23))
 (segment (start 142.9 92.12) (end 146.86 92.13) (width 0.4) (layer F.Cu) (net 23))
 (segment (start 141.44 110.67) (end 141.44 93.58) (width 0.4) (layer F.Cu) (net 23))
 (segment (start 141.44 93.58) (end 142.9 92.12) (width 0.4) (layer F.Cu) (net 23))
 (segment (start 146.29 84.99) (end 147.67 86.37) (width 0.4) (layer F.Cu) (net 23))
 (segment (start 146.29 82.66) (end 146.29 84.99) (width 0.4) (layer F.Cu) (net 23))
 (segment (start 145.02 82.66) (end 145.21 82.66) (width 0.4) (layer B.Cu) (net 24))
 (segment (start 145.02 81.952894) (end 145.862894 81.11) (width 0.4) (layer F.Cu) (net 24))
 (segment (start 145.02 82.66) (end 145.02 81.952894) (width 0.4) (layer F.Cu) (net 24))
 (via (at 150.13 81.11) (size 0.8) (drill 0.4) (layers F.Cu B.Cu) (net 24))
 (segment (start 145.862894 81.11) (end 150.13 81.11) (width 0.4) (layer F.Cu) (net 24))
 (via (at 148.72 86.79) (size 0.8) (drill 0.4) (layers F.Cu B.Cu) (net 24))
 (via (at 146.74 86.79) (size 0.8) (drill 0.4) (layers F.Cu B.Cu) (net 24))
 (segment (start 148.72 86.79) (end 146.74 86.79) (width 0.4) (layer B.Cu) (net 24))
 (segment (start 139.66 109.895) (end 139.66 110.67) (width 0.4) (layer F.Cu) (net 24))
 (segment (start 140.83999 108.71501) (end 139.66 109.895) (width 0.4) (layer F.Cu) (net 24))
 (segment (start 140.839991 93.331467) (end 140.83999 108.71501) (width 0.4) (layer F.Cu) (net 24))
 (segment (start 146.74 86.79) (end 145.89 87.64) (width 0.4) (layer F.Cu) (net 24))
 (segment (start 145.89 87.64) (end 145.89 91.324999) (width 0.4) (layer F.Cu) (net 24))
 (segment (start 145.89 91.324999) (end 145.695634 91.519365) (width 0.4) (layer F.Cu) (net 24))
 (segment (start 145.695634 91.519365) (end 142.652093 91.519365) (width 0.4) (layer F.Cu) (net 24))
 (segment (start 142.652093 91.519365) (end 140.839991 93.331467) (width 0.4) (layer F.Cu) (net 24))
 (segment (start 150.13 84.019998) (end 150.15 84.039998) (width 0.4) (layer B.Cu) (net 24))
 (segment (start 148.72 86.79) (end 150.15 85.36) (width 0.4) (layer F.Cu) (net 24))
 (via (at 150.15 84.039998) (size 0.8) (drill 0.4) (layers F.Cu B.Cu) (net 24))
 (segment (start 150.15 84.605683) (end 150.15 84.039998) (width 0.4) (layer F.Cu) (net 24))
 (segment (start 150.15 85.36) (end 150.15 84.605683) (width 0.4) (layer F.Cu) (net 24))
 (segment (start 150.13 81.11) (end 150.13 84.019998) (width 0.4) (layer B.Cu) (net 24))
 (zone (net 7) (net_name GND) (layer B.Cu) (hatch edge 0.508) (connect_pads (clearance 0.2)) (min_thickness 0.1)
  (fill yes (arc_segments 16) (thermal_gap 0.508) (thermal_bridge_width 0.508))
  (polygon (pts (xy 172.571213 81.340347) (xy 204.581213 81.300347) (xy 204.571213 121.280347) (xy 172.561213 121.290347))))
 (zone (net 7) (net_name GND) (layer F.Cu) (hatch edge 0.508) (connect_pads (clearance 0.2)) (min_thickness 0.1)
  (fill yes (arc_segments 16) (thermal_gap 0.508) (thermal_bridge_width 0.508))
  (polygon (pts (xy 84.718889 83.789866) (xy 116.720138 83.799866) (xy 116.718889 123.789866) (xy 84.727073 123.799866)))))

